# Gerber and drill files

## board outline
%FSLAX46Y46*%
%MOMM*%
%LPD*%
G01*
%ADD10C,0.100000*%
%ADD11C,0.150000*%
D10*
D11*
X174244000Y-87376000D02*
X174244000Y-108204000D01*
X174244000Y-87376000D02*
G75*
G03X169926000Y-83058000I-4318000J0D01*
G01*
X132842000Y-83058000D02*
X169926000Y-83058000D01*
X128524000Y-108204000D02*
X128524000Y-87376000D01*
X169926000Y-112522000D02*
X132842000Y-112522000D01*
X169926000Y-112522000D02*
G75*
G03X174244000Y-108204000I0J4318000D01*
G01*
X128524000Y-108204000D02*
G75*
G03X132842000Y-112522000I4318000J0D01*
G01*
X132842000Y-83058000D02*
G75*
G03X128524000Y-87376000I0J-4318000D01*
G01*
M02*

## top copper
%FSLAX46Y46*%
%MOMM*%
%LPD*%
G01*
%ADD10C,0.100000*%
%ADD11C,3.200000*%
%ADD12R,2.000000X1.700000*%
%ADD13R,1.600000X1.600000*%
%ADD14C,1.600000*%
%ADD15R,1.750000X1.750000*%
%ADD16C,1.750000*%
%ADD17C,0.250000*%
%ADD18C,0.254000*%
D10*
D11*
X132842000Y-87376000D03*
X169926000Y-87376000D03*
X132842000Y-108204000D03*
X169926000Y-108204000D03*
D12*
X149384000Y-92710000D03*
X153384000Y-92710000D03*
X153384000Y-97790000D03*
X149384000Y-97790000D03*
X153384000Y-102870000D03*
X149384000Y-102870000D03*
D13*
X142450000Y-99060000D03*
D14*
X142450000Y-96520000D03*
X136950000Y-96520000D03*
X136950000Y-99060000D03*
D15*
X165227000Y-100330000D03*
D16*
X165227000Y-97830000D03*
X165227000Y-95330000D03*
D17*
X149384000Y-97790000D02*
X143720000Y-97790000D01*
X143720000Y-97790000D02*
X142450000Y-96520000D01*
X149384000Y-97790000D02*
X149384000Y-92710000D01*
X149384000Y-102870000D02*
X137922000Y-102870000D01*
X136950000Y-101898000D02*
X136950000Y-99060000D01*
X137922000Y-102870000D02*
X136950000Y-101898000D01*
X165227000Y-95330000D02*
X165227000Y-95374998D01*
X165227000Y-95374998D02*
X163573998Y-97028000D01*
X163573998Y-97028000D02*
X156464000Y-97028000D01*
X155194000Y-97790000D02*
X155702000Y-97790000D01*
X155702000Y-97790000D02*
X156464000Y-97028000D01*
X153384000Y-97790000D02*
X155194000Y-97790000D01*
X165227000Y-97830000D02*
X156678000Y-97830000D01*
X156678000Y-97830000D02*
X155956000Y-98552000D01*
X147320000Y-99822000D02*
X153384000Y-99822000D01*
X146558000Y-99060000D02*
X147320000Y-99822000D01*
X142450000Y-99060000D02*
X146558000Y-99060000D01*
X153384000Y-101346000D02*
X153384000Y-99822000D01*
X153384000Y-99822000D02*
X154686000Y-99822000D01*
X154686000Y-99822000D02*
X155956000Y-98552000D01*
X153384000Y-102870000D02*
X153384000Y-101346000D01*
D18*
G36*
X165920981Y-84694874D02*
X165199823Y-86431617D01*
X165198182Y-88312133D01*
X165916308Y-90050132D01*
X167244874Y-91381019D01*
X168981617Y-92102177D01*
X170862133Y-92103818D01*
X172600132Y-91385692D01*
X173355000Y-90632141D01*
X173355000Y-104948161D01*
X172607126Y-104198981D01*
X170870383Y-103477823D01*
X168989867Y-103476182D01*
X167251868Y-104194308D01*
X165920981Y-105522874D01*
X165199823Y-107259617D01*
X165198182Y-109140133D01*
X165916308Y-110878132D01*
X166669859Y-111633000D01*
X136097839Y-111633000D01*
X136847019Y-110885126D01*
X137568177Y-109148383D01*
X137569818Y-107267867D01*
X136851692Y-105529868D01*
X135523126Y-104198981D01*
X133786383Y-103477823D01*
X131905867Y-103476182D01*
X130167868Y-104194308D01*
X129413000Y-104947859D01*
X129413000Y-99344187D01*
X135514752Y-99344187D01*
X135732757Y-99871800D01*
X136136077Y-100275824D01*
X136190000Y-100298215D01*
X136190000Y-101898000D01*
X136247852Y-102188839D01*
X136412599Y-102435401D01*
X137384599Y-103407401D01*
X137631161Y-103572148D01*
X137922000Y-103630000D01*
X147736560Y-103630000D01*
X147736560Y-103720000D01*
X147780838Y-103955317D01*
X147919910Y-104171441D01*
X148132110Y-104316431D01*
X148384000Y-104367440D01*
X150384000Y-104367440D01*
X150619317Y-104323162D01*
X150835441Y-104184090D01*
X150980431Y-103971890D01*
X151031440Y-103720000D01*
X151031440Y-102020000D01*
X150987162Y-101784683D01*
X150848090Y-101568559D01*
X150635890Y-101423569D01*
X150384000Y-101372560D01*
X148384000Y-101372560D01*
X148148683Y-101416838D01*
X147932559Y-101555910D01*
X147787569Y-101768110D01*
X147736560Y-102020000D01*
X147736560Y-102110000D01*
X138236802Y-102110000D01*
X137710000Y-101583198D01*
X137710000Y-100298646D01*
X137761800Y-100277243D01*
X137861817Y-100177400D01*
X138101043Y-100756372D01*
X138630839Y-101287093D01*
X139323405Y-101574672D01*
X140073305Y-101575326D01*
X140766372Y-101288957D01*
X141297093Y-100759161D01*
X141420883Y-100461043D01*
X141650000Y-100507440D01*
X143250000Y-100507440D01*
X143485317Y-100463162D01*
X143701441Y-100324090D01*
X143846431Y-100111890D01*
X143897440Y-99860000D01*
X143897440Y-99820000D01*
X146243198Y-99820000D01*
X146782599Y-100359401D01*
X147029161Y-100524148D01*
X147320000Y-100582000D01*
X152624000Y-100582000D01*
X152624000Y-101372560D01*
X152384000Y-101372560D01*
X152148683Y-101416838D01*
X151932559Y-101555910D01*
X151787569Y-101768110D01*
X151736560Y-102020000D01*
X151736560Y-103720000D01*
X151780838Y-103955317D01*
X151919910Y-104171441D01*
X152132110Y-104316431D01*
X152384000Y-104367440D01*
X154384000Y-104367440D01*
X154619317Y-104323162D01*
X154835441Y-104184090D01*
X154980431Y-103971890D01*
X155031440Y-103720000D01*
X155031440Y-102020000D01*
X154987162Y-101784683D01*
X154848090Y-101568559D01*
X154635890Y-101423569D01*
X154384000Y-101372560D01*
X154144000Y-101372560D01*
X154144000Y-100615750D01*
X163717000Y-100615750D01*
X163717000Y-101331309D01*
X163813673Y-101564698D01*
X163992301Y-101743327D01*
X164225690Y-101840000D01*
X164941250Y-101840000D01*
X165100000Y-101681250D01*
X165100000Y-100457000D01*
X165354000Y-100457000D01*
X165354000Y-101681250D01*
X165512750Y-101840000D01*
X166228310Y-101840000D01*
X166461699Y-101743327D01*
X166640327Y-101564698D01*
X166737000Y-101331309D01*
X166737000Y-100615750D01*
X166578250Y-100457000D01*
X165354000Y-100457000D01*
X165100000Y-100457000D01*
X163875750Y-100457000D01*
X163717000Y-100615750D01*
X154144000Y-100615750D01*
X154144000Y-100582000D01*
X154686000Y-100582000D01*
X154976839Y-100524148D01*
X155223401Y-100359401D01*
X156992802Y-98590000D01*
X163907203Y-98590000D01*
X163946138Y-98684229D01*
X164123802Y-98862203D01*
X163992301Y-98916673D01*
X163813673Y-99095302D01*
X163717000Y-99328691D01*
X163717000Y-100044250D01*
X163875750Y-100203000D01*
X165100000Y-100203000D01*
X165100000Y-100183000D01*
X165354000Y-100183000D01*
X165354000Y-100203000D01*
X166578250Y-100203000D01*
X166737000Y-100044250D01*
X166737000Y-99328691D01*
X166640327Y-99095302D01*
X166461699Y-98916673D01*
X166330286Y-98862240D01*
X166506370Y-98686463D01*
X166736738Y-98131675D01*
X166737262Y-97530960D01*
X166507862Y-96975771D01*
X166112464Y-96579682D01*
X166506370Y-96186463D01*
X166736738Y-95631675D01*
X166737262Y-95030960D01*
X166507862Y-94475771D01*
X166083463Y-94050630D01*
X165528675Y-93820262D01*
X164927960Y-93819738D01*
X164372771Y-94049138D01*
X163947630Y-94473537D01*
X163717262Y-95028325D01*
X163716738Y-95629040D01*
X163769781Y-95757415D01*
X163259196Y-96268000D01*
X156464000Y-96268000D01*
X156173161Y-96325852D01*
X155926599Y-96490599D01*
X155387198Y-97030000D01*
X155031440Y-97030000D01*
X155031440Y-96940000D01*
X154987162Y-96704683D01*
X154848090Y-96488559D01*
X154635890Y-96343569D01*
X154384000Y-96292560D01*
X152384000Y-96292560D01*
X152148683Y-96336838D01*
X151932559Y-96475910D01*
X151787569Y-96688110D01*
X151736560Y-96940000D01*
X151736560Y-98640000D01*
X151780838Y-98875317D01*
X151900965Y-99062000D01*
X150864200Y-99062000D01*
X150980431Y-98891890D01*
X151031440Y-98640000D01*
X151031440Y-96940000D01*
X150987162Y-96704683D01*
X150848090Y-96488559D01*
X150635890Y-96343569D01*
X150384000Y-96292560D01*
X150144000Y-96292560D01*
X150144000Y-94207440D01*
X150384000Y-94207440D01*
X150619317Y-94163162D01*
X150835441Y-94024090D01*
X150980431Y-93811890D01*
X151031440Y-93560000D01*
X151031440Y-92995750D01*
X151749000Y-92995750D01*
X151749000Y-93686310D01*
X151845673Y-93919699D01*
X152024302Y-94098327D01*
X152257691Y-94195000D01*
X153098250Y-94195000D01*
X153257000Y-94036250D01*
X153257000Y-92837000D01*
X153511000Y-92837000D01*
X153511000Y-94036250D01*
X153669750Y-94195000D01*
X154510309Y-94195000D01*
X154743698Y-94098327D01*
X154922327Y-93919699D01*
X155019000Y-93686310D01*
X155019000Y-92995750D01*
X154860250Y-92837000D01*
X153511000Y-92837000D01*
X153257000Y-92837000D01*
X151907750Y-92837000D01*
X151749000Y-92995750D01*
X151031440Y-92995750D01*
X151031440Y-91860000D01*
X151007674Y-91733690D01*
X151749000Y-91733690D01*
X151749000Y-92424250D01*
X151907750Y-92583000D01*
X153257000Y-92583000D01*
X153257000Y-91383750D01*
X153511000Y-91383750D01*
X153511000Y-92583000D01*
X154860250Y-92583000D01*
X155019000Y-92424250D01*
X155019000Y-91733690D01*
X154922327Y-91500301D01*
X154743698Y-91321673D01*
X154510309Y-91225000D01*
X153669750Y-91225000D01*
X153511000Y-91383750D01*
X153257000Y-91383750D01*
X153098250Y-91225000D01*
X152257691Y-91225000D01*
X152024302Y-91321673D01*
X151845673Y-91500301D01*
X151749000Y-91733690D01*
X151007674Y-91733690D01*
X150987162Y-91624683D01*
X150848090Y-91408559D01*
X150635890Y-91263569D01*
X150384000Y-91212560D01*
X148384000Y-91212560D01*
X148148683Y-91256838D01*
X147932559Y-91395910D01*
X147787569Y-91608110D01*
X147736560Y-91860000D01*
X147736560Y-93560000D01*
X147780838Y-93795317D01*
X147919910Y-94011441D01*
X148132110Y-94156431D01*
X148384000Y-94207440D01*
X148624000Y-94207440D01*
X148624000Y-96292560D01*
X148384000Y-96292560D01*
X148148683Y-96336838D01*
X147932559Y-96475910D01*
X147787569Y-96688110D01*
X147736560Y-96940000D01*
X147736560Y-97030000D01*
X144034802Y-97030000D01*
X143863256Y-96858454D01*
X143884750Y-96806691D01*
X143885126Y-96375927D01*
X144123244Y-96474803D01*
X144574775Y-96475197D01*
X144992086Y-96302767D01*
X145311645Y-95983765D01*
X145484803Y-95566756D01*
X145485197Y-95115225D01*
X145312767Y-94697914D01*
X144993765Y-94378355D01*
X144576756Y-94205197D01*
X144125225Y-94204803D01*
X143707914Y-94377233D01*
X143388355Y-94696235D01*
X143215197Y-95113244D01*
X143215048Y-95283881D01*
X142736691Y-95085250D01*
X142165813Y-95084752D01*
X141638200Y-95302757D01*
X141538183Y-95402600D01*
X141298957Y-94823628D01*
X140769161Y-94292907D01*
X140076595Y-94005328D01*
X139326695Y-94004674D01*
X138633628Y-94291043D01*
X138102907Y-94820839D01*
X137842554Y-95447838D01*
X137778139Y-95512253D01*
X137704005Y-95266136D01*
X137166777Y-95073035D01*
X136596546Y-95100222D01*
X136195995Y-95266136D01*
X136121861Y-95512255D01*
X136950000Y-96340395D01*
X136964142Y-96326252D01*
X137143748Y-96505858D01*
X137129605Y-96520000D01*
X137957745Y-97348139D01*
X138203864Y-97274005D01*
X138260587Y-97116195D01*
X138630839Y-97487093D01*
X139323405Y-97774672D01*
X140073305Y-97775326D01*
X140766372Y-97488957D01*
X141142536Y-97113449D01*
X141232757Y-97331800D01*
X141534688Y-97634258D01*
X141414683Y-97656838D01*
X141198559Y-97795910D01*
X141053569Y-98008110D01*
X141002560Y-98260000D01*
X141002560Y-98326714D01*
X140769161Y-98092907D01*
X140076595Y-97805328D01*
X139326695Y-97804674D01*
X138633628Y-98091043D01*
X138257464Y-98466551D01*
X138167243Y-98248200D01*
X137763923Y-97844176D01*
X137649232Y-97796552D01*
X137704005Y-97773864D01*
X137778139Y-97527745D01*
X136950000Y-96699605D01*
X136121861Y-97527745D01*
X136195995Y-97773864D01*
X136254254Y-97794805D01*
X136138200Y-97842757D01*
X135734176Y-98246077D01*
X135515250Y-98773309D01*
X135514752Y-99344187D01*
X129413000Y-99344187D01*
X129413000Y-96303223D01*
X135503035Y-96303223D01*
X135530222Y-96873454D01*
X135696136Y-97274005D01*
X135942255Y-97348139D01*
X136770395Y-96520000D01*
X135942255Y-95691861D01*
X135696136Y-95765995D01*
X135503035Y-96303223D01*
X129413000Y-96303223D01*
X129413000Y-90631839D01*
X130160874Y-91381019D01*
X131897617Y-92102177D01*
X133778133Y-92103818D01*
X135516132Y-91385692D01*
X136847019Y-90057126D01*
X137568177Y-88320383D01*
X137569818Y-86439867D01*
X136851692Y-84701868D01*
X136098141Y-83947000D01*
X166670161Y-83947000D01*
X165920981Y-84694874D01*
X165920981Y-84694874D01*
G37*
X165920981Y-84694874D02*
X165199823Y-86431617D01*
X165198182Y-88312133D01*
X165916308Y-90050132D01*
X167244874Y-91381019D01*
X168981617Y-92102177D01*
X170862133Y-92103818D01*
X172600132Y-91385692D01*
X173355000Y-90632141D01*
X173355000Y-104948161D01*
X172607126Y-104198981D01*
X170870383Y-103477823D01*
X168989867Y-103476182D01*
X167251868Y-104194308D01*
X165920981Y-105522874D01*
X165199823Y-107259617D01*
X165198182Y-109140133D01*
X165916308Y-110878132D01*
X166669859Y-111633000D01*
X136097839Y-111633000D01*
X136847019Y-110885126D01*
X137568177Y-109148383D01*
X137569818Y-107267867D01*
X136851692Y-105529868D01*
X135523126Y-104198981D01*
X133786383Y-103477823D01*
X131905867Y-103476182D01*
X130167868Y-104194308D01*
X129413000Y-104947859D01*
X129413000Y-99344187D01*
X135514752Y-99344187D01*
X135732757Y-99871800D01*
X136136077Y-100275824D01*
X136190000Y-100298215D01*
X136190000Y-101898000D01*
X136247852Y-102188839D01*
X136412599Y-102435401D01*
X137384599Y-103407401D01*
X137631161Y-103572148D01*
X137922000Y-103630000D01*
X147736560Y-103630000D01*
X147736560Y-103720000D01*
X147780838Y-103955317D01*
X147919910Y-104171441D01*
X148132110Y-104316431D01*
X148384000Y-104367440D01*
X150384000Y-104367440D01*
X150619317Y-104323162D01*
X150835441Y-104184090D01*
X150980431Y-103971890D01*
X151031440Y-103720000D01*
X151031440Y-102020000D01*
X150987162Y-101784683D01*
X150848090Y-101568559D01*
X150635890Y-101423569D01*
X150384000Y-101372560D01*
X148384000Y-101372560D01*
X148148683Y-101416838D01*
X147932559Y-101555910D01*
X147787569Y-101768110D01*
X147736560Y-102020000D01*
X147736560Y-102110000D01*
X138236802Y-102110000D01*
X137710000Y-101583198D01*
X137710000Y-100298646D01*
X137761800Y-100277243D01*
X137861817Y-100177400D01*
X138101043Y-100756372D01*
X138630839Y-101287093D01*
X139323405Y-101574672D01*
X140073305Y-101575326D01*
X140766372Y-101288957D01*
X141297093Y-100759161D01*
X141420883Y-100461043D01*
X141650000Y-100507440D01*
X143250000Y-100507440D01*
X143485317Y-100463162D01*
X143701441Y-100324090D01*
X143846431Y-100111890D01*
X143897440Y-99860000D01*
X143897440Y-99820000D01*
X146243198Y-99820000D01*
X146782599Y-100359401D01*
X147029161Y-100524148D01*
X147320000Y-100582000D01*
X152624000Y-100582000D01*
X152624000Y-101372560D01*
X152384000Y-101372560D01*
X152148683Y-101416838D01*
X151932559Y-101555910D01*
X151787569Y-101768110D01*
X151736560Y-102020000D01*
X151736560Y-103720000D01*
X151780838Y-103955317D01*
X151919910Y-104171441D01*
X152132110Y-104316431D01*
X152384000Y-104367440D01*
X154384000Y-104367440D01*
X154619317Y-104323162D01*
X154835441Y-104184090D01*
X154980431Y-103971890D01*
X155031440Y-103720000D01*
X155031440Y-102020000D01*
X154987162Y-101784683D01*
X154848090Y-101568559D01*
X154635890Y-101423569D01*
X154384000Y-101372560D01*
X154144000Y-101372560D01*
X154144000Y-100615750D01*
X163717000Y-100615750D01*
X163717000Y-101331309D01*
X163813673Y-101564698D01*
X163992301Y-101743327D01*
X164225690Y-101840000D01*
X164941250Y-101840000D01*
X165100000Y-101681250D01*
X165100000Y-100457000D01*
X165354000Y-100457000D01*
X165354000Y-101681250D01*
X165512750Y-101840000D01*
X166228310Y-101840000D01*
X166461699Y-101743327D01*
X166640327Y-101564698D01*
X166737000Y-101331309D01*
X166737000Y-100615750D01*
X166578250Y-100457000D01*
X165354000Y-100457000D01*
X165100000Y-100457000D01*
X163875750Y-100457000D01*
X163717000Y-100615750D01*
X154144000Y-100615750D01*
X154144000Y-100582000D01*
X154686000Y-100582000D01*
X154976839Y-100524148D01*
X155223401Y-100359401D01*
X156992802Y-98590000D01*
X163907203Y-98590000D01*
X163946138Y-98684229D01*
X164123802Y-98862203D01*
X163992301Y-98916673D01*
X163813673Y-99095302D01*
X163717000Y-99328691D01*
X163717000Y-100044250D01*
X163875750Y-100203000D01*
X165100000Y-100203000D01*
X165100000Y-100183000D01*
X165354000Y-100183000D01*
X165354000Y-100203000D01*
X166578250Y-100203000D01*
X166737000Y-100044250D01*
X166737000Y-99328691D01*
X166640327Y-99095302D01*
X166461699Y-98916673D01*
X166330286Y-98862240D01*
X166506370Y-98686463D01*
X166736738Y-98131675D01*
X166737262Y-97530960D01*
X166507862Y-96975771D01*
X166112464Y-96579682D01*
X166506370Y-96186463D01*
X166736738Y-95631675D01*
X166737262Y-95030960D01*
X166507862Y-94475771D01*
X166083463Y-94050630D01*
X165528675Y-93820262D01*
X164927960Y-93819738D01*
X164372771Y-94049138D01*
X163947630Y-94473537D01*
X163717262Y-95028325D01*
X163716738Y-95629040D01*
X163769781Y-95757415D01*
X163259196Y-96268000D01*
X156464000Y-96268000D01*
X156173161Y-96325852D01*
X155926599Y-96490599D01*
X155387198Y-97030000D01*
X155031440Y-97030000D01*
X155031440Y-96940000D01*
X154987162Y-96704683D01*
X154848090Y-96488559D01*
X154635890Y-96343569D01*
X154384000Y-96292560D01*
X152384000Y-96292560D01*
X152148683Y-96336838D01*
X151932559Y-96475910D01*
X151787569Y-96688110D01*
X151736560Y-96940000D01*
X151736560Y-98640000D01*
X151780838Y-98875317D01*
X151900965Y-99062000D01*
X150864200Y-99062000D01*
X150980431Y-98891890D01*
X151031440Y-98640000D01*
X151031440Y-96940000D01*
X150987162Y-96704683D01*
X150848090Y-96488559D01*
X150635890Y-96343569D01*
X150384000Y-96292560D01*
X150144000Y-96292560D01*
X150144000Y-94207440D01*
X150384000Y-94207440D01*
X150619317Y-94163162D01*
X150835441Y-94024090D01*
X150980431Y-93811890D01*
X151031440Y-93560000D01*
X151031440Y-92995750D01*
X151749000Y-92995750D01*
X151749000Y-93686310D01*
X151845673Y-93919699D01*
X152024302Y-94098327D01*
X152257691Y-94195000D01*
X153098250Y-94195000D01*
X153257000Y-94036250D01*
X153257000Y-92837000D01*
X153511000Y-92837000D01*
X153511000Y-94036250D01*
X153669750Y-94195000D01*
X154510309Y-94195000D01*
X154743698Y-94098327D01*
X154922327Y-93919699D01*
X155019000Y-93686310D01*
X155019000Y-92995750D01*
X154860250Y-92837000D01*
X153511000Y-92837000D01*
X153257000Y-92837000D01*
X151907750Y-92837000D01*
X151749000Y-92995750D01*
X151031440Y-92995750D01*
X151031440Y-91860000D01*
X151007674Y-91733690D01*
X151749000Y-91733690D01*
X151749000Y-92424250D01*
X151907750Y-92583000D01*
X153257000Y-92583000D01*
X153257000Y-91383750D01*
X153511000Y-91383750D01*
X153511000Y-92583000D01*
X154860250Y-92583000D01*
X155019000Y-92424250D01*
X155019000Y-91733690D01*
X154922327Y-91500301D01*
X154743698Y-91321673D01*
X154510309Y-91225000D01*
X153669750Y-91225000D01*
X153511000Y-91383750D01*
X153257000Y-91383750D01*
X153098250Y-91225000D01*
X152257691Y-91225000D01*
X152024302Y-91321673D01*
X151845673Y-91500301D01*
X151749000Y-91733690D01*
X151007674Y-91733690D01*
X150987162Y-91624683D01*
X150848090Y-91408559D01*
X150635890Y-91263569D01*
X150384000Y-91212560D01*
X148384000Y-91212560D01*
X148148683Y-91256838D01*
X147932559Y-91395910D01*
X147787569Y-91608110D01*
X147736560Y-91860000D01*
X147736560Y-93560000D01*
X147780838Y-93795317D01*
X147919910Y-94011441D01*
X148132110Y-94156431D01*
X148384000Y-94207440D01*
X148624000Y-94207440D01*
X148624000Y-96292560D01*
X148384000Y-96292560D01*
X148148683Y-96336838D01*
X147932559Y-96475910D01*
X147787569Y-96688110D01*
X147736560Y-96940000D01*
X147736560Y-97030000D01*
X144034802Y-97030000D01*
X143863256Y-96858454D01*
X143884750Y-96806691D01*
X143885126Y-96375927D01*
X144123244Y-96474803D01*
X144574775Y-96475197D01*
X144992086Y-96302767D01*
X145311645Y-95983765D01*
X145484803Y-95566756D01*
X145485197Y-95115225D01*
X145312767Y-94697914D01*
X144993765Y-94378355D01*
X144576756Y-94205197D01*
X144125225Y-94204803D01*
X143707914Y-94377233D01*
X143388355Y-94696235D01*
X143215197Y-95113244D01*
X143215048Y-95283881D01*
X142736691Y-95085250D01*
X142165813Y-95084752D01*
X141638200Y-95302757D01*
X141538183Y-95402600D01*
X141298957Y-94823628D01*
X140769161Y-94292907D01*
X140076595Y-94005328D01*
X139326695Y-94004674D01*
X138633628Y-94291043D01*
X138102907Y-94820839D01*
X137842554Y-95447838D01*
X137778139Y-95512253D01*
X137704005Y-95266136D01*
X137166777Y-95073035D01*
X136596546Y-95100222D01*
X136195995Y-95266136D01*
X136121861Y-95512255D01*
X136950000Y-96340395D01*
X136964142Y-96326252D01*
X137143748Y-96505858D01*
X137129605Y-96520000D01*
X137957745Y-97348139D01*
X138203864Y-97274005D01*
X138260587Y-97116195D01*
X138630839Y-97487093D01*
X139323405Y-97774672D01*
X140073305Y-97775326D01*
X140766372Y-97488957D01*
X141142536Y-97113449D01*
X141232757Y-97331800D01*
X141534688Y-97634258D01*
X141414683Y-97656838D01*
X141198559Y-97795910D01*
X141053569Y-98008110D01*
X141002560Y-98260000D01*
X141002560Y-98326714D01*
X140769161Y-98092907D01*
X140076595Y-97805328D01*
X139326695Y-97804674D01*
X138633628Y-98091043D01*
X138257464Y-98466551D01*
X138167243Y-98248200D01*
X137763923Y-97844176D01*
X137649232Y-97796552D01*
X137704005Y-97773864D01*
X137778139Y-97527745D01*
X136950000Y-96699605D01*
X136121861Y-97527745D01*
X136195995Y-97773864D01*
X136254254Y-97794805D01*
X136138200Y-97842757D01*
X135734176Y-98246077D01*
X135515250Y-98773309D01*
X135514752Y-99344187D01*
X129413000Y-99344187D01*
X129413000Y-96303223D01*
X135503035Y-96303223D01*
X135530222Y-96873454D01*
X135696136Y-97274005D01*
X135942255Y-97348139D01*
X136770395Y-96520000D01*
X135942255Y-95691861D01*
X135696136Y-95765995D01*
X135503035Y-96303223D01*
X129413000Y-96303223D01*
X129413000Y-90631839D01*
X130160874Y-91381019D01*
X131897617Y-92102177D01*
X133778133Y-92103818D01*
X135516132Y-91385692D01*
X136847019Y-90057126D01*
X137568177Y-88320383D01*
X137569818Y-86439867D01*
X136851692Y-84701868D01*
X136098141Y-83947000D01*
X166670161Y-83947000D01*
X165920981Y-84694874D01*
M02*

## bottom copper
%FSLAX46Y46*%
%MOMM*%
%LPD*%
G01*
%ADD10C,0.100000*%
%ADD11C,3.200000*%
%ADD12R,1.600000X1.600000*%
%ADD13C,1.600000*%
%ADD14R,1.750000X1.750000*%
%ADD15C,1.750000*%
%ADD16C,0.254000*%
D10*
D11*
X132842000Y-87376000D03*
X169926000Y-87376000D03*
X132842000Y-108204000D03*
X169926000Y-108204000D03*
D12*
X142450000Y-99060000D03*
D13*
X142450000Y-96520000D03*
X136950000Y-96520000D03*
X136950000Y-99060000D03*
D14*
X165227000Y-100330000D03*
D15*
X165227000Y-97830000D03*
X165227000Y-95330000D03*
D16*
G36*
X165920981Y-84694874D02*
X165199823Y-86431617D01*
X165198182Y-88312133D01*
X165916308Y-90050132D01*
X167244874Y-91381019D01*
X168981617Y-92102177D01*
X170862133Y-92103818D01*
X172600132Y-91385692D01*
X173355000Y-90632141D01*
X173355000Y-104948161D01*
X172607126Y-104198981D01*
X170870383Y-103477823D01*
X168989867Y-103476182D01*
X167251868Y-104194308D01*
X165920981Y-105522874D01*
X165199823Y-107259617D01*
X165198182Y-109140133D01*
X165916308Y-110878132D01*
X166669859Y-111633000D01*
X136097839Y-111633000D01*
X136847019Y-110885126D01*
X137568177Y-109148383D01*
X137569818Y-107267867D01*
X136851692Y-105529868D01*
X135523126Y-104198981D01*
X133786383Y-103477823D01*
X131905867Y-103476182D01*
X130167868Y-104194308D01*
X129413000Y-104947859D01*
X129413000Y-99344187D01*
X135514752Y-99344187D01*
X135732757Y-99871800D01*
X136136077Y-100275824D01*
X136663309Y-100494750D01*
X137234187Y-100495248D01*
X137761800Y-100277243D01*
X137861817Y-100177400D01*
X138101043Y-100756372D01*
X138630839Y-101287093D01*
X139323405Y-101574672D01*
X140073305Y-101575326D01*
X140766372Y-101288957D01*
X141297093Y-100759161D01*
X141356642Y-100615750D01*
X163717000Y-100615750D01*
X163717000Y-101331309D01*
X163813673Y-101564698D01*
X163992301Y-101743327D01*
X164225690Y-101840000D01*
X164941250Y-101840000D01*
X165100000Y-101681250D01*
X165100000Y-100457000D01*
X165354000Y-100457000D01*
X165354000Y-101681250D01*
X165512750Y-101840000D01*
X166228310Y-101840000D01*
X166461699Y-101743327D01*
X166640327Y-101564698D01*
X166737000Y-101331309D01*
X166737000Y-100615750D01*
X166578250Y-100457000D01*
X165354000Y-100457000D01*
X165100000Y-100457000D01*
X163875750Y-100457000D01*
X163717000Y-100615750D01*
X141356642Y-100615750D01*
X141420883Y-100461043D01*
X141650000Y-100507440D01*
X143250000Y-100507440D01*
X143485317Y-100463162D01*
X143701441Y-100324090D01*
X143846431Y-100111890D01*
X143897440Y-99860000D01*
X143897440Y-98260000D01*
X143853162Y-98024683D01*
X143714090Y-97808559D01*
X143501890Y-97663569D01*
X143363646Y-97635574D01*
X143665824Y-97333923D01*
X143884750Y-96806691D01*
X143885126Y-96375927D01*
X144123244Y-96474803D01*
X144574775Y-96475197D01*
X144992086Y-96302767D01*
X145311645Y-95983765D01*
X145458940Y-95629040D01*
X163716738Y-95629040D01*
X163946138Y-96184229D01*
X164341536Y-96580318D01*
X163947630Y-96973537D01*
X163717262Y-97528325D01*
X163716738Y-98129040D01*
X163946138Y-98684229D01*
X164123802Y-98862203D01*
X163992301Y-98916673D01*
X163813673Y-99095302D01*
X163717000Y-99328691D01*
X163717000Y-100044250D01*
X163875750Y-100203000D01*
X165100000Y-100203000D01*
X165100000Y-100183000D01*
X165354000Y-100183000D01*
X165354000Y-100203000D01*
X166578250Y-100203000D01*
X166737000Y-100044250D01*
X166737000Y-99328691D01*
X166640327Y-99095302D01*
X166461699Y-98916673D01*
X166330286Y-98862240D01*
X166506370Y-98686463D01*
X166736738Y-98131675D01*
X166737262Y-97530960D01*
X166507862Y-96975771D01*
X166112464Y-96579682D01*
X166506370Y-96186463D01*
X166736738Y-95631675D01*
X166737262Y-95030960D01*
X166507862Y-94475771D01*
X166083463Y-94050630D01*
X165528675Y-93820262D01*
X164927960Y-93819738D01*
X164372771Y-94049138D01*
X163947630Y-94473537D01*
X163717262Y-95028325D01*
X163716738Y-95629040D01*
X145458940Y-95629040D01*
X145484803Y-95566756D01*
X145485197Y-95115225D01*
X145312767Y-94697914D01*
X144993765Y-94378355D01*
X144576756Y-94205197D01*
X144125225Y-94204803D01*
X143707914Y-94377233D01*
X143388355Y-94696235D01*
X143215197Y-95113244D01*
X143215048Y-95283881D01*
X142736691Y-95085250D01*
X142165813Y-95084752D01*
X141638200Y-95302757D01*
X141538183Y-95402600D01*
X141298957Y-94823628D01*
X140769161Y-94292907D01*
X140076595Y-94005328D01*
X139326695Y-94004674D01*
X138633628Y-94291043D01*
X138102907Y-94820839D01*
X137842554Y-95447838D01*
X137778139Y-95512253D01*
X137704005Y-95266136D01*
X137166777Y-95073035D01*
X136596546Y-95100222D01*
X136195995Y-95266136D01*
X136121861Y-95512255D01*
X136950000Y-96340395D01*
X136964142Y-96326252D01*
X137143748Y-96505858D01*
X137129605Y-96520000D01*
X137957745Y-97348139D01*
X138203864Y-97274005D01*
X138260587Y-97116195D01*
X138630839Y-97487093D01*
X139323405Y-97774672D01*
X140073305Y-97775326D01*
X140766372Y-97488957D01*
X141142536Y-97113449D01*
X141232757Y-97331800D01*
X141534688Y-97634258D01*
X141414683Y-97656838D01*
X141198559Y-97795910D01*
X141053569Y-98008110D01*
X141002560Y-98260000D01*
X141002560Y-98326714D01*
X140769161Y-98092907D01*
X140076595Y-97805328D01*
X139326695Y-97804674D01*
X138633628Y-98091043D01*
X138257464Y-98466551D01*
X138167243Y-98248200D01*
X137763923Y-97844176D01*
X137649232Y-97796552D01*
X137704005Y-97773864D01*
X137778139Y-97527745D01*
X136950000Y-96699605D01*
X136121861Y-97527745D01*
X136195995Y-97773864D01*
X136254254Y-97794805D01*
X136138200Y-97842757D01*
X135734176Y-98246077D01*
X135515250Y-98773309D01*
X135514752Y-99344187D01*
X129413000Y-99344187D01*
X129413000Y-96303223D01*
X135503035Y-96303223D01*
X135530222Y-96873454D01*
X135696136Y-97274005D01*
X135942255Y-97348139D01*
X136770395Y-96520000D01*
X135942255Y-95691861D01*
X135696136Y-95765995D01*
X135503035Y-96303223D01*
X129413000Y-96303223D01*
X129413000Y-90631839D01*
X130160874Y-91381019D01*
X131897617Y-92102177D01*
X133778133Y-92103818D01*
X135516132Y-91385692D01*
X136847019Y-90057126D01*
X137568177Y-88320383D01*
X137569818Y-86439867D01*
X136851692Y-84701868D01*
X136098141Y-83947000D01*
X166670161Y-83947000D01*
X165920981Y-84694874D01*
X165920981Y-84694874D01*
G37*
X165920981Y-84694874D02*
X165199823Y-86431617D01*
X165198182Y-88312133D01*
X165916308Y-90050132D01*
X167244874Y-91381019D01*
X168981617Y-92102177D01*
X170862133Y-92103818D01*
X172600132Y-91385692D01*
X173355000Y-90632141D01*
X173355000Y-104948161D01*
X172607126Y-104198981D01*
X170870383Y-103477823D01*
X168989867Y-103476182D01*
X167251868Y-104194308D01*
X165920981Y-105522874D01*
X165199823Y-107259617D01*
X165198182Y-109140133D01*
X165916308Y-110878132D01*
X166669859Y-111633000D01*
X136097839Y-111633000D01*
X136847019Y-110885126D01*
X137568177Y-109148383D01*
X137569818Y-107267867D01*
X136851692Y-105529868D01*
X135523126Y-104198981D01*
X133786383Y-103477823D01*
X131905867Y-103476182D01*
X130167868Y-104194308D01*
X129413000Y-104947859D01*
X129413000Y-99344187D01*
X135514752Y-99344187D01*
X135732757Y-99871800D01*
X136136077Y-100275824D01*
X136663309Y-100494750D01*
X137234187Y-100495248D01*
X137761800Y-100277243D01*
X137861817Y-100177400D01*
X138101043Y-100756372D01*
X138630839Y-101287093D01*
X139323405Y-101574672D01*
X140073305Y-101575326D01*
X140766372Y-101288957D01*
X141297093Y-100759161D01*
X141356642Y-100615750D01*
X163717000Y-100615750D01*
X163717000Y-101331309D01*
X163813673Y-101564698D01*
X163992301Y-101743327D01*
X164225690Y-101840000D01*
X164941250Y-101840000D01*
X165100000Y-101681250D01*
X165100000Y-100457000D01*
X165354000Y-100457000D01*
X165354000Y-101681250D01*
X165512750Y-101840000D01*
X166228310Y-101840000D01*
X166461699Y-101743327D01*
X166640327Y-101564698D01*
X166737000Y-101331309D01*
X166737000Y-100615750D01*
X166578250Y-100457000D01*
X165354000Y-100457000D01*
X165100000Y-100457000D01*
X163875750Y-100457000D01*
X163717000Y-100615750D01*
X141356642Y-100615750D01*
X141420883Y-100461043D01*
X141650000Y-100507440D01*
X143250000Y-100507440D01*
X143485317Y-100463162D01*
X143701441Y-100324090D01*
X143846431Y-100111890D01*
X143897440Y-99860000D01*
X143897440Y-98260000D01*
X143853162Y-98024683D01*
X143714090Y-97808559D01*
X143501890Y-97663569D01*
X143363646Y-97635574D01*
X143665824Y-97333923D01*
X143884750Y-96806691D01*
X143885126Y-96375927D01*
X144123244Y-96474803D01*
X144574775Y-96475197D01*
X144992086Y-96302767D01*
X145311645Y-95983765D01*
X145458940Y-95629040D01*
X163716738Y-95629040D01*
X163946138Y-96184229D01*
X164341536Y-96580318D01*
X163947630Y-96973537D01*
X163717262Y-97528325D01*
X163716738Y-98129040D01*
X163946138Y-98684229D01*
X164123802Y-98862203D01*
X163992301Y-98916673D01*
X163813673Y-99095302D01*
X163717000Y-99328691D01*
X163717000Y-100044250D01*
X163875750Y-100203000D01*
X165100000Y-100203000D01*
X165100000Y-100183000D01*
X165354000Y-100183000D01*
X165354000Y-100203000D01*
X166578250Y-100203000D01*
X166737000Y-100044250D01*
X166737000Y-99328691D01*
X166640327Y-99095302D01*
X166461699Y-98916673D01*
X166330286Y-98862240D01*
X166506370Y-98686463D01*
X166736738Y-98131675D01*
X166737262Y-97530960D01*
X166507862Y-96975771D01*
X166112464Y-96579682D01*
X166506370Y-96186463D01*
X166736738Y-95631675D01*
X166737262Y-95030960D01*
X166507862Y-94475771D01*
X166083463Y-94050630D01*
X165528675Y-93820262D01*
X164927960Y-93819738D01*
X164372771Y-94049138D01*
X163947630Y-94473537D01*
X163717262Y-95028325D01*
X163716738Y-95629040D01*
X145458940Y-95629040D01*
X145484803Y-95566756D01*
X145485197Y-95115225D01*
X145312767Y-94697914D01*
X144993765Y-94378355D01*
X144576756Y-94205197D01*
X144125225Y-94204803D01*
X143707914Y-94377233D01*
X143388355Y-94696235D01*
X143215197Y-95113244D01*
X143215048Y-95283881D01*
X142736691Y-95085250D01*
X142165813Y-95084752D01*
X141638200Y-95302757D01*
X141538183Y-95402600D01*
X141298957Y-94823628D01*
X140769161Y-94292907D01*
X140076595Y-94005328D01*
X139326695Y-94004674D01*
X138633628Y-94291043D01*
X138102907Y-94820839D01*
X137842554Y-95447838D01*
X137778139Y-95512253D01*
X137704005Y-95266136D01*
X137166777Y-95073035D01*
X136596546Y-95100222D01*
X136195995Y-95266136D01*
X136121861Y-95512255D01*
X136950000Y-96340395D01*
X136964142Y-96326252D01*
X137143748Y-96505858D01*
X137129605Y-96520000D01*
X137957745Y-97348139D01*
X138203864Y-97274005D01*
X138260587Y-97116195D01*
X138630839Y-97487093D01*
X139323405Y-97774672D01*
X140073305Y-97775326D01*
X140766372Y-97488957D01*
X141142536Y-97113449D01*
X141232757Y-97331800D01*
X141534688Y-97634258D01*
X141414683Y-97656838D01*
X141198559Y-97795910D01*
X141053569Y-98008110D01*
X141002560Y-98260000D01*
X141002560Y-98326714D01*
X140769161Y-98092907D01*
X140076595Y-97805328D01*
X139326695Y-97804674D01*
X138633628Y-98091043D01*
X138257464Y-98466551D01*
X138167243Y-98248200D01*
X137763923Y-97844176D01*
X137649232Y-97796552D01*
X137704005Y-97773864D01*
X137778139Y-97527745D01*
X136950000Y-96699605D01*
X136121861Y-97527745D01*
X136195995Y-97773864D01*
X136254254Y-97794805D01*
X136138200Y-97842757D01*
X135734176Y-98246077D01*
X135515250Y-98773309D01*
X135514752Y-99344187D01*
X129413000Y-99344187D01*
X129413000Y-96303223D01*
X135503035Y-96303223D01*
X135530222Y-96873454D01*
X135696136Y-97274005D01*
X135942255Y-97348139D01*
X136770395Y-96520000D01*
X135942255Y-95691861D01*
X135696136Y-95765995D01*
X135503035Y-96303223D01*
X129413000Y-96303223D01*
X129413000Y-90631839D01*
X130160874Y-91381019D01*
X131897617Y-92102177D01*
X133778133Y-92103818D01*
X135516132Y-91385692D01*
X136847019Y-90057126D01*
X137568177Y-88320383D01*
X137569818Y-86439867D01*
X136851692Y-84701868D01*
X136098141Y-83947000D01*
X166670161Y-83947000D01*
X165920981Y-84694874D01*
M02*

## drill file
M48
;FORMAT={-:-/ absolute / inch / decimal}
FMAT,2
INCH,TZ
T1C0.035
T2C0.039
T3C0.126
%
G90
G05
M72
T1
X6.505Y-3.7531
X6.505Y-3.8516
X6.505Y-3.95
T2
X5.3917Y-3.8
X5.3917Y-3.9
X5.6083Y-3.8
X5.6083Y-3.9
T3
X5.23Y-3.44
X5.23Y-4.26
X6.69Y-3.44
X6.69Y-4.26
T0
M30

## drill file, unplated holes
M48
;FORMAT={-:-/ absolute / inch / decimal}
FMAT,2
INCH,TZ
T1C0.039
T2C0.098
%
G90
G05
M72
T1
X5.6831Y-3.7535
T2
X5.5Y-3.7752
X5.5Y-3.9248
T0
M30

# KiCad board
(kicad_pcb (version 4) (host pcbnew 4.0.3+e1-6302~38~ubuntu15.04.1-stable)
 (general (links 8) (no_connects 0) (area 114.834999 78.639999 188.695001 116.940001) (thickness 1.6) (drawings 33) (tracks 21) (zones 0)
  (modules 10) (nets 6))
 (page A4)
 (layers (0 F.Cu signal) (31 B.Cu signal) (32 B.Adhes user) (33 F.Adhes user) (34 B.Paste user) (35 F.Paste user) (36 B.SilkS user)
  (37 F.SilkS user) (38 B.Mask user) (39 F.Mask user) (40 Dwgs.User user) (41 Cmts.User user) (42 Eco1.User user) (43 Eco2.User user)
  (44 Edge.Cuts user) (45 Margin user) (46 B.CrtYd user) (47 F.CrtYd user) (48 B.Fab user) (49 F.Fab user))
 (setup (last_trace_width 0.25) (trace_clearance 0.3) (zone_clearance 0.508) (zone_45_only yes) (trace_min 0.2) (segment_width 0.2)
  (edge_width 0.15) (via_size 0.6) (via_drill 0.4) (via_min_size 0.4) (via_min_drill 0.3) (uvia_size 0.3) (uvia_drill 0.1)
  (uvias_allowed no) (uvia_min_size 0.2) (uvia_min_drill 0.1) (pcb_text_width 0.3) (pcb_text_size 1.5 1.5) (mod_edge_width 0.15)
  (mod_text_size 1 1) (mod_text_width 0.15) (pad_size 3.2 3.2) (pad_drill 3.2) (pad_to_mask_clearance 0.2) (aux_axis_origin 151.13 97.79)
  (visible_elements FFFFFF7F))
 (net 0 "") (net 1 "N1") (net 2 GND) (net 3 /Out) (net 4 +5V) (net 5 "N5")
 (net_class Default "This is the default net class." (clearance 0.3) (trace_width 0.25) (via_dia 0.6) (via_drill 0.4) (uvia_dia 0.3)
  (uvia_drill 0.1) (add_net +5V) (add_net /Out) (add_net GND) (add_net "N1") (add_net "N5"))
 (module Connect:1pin (layer F.Cu) (at 132.842 87.376)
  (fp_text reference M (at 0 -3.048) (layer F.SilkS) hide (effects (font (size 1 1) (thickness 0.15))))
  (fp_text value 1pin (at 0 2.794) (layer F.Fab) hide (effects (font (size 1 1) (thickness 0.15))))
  (pad 1 thru_hole circle (at 0 0) (size 3.2 3.2) (drill 3.2) (layers *.Cu *.Mask F.SilkS) (solder_mask_margin 2) (clearance 3)))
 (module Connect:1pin (layer F.Cu) (at 169.926 87.376)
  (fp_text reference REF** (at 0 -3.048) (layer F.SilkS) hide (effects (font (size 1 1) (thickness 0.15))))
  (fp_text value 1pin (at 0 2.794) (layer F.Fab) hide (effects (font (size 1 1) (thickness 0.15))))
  (pad 1 thru_hole circle (at 0 0) (size 3.2 3.2) (drill 3.2) (layers *.Cu *.Mask F.SilkS) (solder_mask_margin 2) (clearance 3)))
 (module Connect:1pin (layer F.Cu) (at 132.842 108.204)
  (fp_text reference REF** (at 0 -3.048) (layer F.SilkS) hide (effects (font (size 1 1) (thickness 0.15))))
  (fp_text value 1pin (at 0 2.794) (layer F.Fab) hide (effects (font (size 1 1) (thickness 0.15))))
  (pad 1 thru_hole circle (at 0 0) (size 3.2 3.2) (drill 3.2) (layers *.Cu *.Mask F.SilkS) (solder_mask_margin 2) (clearance 3)))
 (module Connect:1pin (layer F.Cu) (at 169.926 108.204)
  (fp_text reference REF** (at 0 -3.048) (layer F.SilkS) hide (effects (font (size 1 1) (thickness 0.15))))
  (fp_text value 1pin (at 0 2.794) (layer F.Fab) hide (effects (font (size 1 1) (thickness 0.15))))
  (pad 1 thru_hole circle (at 0 0) (size 3.2 3.2) (drill 3.2) (layers *.Cu *.Mask F.SilkS) (solder_mask_margin 2) (clearance 3)))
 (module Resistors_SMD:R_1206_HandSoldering (layer F.Cu) (at 151.384 92.71)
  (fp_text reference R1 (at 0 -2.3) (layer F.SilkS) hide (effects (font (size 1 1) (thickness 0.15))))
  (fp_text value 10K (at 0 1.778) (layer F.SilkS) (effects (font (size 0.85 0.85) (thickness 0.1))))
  (pad 1 smd rect (at -2 0) (size 2 1.7) (layers F.Cu F.Paste F.Mask) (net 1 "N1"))
  (pad 2 smd rect (at 2 0) (size 2 1.7) (layers F.Cu F.Paste F.Mask) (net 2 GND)))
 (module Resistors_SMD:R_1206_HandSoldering (layer F.Cu) (at 151.384 97.79 180)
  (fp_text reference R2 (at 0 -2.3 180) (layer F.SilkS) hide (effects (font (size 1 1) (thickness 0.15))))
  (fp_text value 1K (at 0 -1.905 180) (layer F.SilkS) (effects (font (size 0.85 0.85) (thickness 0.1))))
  (pad 1 smd rect (at -2 0 180) (size 2 1.7) (layers F.Cu F.Paste F.Mask) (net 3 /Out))
  (pad 2 smd rect (at 2 0 180) (size 2 1.7) (layers F.Cu F.Paste F.Mask) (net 1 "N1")))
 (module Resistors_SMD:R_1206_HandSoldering (layer F.Cu) (at 151.384 102.87 180)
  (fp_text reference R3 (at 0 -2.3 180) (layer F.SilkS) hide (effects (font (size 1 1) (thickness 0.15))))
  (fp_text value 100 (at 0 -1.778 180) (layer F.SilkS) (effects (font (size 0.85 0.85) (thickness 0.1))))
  (pad 1 smd rect (at -2 0 180) (size 2 1.7) (layers F.Cu F.Paste F.Mask) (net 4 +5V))
  (pad 2 smd rect (at 2 0 180) (size 2 1.7) (layers F.Cu F.Paste F.Mask) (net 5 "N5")))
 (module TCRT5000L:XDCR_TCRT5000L (layer F.Cu) (at 139.7 97.79 180) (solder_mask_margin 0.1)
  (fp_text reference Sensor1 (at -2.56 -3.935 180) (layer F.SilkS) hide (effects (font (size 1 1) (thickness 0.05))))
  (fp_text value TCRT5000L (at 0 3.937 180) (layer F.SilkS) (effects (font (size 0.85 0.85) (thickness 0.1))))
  (pad 1 thru_hole rect (at -2.75 -1.27 180) (size 1.6 1.6) (drill 1) (layers *.Cu *.Mask F.SilkS) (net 4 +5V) (solder_mask_margin 0.2))
  (pad 2 thru_hole circle (at -2.75 1.27 180) (size 1.6 1.6) (drill 1) (layers *.Cu *.Mask F.SilkS) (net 1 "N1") (solder_mask_margin 0.2))
  (pad 3 thru_hole circle (at 2.75 1.27 180) (size 1.6 1.6) (drill 1) (layers *.Cu *.Mask F.SilkS) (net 2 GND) (solder_mask_margin 0.2))
  (pad 4 thru_hole circle (at 2.75 -1.27 180) (size 1.6 1.6) (drill 1) (layers *.Cu *.Mask F.SilkS) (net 5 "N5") (solder_mask_margin 0.2))
  (pad Hole np_thru_hole circle (at 0 -1.9 180) (size 2.5 2.5) (drill 2.5) (layers))
  (pad Hole np_thru_hole circle (at 0 1.9 180) (size 2.5 2.5) (drill 2.5) (layers))
  (pad Hole np_thru_hole circle (at -4.65 2.45 180) (size 1 1) (drill 1) (layers)))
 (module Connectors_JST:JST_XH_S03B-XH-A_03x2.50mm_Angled (layer F.Cu) (at 165.227 100.33 90)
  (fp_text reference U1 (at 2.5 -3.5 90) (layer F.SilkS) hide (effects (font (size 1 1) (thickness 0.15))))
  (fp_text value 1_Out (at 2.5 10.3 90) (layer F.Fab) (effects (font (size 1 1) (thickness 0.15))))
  (pad 1 thru_hole rect (at 0 0 90) (size 1.75 1.75) (drill 0.9) (layers *.Cu *.Mask F.SilkS) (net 2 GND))
  (pad 2 thru_hole circle (at 2.5 0 90) (size 1.75 1.75) (drill 0.9) (layers *.Cu *.Mask F.SilkS) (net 4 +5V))
  (pad 3 thru_hole circle (at 5 0 90) (size 1.75 1.75) (drill 0.9) (layers *.Cu *.Mask F.SilkS) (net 3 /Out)))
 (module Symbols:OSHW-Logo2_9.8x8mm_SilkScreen (layer B.Cu) (at 151.384 97.79 180)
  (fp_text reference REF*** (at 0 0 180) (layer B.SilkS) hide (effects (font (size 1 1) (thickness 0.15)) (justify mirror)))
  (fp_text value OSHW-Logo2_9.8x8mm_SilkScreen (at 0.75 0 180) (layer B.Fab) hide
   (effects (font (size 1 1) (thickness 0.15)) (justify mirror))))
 (gr_line (start 174.244 87.376) (end 174.244 108.204) (angle 90) (layer Edge.Cuts) (width 0.15))
 (gr_arc (start 169.926 87.376) (end 169.926 83.058) (angle 90) (layer Edge.Cuts) (width 0.15))
 (gr_line (start 132.842 83.058) (end 169.926 83.058) (angle 90) (layer Edge.Cuts) (width 0.15))
 (gr_line (start 128.524 108.204) (end 128.524 87.376) (angle 90) (layer Edge.Cuts) (width 0.15))
 (gr_line (start 169.926 112.522) (end 132.842 112.522) (angle 90) (layer Edge.Cuts) (width 0.15))
 (gr_arc (start 169.926 108.204) (end 174.244 108.204) (angle 90) (layer Edge.Cuts) (width 0.15))
 (gr_arc (start 132.842 108.204) (end 132.842 112.522) (angle 90) (layer Edge.Cuts) (width 0.15))
 (gr_arc (start 132.842 87.376) (end 128.524 87.376) (angle 90) (layer Edge.Cuts) (width 0.15))
 (segment (start 149.384 97.79) (end 143.72 97.79) (width 0.25) (layer F.Cu) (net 1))
 (segment (start 143.72 97.79) (end 142.45 96.52) (width 0.25) (layer F.Cu) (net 1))
 (segment (start 149.384 97.79) (end 149.384 92.71) (width 0.25) (layer F.Cu) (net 1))
 (segment (start 149.384 102.87) (end 137.922 102.87) (width 0.25) (layer F.Cu) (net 5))
 (segment (start 136.95 101.898) (end 136.95 99.06) (width 0.25) (layer F.Cu) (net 5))
 (segment (start 137.922 102.87) (end 136.95 101.898) (width 0.25) (layer F.Cu) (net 5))
 (segment (start 165.227 95.33) (end 165.227 95.374998) (width 0.25) (layer F.Cu) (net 3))
 (segment (start 165.227 95.374998) (end 163.573998 97.028) (width 0.25) (layer F.Cu) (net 3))
 (segment (start 163.573998 97.028) (end 156.464 97.028) (width 0.25) (layer F.Cu) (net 3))
 (segment (start 155.194 97.79) (end 155.702 97.79) (width 0.25) (layer F.Cu) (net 3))
 (segment (start 155.702 97.79) (end 156.464 97.028) (width 0.25) (layer F.Cu) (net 3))
 (segment (start 153.384 97.79) (end 155.194 97.79) (width 0.25) (layer F.Cu) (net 3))
 (segment (start 165.227 97.83) (end 156.678 97.83) (width 0.25) (layer F.Cu) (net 4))
 (segment (start 156.678 97.83) (end 155.956 98.552) (width 0.25) (layer F.Cu) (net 4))
 (segment (start 147.32 99.822) (end 153.384 99.822) (width 0.25) (layer F.Cu) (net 4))
 (segment (start 146.558 99.06) (end 147.32 99.822) (width 0.25) (layer F.Cu) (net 4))
 (segment (start 142.45 99.06) (end 146.558 99.06) (width 0.25) (layer F.Cu) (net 4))
 (segment (start 153.384 101.346) (end 153.384 99.822) (width 0.25) (layer F.Cu) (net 4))
 (segment (start 153.384 99.822) (end 154.686 99.822) (width 0.25) (layer F.Cu) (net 4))
 (segment (start 154.686 99.822) (end 155.956 98.552) (width 0.25) (layer F.Cu) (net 4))
 (segment (start 153.384 102.87) (end 153.384 101.346) (width 0.25) (layer F.Cu) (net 4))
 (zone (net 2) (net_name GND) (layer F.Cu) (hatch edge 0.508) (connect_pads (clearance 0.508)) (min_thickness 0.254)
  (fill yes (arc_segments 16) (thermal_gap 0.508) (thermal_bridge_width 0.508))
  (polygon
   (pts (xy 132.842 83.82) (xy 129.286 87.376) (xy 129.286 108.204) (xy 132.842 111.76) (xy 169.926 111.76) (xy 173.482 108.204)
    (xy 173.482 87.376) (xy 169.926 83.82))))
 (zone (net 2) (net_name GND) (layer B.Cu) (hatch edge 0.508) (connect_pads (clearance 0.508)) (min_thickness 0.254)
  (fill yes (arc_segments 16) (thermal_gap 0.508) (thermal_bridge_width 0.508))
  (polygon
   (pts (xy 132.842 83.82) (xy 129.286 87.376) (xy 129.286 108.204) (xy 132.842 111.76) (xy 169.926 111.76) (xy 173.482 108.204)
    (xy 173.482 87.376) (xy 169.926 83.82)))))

